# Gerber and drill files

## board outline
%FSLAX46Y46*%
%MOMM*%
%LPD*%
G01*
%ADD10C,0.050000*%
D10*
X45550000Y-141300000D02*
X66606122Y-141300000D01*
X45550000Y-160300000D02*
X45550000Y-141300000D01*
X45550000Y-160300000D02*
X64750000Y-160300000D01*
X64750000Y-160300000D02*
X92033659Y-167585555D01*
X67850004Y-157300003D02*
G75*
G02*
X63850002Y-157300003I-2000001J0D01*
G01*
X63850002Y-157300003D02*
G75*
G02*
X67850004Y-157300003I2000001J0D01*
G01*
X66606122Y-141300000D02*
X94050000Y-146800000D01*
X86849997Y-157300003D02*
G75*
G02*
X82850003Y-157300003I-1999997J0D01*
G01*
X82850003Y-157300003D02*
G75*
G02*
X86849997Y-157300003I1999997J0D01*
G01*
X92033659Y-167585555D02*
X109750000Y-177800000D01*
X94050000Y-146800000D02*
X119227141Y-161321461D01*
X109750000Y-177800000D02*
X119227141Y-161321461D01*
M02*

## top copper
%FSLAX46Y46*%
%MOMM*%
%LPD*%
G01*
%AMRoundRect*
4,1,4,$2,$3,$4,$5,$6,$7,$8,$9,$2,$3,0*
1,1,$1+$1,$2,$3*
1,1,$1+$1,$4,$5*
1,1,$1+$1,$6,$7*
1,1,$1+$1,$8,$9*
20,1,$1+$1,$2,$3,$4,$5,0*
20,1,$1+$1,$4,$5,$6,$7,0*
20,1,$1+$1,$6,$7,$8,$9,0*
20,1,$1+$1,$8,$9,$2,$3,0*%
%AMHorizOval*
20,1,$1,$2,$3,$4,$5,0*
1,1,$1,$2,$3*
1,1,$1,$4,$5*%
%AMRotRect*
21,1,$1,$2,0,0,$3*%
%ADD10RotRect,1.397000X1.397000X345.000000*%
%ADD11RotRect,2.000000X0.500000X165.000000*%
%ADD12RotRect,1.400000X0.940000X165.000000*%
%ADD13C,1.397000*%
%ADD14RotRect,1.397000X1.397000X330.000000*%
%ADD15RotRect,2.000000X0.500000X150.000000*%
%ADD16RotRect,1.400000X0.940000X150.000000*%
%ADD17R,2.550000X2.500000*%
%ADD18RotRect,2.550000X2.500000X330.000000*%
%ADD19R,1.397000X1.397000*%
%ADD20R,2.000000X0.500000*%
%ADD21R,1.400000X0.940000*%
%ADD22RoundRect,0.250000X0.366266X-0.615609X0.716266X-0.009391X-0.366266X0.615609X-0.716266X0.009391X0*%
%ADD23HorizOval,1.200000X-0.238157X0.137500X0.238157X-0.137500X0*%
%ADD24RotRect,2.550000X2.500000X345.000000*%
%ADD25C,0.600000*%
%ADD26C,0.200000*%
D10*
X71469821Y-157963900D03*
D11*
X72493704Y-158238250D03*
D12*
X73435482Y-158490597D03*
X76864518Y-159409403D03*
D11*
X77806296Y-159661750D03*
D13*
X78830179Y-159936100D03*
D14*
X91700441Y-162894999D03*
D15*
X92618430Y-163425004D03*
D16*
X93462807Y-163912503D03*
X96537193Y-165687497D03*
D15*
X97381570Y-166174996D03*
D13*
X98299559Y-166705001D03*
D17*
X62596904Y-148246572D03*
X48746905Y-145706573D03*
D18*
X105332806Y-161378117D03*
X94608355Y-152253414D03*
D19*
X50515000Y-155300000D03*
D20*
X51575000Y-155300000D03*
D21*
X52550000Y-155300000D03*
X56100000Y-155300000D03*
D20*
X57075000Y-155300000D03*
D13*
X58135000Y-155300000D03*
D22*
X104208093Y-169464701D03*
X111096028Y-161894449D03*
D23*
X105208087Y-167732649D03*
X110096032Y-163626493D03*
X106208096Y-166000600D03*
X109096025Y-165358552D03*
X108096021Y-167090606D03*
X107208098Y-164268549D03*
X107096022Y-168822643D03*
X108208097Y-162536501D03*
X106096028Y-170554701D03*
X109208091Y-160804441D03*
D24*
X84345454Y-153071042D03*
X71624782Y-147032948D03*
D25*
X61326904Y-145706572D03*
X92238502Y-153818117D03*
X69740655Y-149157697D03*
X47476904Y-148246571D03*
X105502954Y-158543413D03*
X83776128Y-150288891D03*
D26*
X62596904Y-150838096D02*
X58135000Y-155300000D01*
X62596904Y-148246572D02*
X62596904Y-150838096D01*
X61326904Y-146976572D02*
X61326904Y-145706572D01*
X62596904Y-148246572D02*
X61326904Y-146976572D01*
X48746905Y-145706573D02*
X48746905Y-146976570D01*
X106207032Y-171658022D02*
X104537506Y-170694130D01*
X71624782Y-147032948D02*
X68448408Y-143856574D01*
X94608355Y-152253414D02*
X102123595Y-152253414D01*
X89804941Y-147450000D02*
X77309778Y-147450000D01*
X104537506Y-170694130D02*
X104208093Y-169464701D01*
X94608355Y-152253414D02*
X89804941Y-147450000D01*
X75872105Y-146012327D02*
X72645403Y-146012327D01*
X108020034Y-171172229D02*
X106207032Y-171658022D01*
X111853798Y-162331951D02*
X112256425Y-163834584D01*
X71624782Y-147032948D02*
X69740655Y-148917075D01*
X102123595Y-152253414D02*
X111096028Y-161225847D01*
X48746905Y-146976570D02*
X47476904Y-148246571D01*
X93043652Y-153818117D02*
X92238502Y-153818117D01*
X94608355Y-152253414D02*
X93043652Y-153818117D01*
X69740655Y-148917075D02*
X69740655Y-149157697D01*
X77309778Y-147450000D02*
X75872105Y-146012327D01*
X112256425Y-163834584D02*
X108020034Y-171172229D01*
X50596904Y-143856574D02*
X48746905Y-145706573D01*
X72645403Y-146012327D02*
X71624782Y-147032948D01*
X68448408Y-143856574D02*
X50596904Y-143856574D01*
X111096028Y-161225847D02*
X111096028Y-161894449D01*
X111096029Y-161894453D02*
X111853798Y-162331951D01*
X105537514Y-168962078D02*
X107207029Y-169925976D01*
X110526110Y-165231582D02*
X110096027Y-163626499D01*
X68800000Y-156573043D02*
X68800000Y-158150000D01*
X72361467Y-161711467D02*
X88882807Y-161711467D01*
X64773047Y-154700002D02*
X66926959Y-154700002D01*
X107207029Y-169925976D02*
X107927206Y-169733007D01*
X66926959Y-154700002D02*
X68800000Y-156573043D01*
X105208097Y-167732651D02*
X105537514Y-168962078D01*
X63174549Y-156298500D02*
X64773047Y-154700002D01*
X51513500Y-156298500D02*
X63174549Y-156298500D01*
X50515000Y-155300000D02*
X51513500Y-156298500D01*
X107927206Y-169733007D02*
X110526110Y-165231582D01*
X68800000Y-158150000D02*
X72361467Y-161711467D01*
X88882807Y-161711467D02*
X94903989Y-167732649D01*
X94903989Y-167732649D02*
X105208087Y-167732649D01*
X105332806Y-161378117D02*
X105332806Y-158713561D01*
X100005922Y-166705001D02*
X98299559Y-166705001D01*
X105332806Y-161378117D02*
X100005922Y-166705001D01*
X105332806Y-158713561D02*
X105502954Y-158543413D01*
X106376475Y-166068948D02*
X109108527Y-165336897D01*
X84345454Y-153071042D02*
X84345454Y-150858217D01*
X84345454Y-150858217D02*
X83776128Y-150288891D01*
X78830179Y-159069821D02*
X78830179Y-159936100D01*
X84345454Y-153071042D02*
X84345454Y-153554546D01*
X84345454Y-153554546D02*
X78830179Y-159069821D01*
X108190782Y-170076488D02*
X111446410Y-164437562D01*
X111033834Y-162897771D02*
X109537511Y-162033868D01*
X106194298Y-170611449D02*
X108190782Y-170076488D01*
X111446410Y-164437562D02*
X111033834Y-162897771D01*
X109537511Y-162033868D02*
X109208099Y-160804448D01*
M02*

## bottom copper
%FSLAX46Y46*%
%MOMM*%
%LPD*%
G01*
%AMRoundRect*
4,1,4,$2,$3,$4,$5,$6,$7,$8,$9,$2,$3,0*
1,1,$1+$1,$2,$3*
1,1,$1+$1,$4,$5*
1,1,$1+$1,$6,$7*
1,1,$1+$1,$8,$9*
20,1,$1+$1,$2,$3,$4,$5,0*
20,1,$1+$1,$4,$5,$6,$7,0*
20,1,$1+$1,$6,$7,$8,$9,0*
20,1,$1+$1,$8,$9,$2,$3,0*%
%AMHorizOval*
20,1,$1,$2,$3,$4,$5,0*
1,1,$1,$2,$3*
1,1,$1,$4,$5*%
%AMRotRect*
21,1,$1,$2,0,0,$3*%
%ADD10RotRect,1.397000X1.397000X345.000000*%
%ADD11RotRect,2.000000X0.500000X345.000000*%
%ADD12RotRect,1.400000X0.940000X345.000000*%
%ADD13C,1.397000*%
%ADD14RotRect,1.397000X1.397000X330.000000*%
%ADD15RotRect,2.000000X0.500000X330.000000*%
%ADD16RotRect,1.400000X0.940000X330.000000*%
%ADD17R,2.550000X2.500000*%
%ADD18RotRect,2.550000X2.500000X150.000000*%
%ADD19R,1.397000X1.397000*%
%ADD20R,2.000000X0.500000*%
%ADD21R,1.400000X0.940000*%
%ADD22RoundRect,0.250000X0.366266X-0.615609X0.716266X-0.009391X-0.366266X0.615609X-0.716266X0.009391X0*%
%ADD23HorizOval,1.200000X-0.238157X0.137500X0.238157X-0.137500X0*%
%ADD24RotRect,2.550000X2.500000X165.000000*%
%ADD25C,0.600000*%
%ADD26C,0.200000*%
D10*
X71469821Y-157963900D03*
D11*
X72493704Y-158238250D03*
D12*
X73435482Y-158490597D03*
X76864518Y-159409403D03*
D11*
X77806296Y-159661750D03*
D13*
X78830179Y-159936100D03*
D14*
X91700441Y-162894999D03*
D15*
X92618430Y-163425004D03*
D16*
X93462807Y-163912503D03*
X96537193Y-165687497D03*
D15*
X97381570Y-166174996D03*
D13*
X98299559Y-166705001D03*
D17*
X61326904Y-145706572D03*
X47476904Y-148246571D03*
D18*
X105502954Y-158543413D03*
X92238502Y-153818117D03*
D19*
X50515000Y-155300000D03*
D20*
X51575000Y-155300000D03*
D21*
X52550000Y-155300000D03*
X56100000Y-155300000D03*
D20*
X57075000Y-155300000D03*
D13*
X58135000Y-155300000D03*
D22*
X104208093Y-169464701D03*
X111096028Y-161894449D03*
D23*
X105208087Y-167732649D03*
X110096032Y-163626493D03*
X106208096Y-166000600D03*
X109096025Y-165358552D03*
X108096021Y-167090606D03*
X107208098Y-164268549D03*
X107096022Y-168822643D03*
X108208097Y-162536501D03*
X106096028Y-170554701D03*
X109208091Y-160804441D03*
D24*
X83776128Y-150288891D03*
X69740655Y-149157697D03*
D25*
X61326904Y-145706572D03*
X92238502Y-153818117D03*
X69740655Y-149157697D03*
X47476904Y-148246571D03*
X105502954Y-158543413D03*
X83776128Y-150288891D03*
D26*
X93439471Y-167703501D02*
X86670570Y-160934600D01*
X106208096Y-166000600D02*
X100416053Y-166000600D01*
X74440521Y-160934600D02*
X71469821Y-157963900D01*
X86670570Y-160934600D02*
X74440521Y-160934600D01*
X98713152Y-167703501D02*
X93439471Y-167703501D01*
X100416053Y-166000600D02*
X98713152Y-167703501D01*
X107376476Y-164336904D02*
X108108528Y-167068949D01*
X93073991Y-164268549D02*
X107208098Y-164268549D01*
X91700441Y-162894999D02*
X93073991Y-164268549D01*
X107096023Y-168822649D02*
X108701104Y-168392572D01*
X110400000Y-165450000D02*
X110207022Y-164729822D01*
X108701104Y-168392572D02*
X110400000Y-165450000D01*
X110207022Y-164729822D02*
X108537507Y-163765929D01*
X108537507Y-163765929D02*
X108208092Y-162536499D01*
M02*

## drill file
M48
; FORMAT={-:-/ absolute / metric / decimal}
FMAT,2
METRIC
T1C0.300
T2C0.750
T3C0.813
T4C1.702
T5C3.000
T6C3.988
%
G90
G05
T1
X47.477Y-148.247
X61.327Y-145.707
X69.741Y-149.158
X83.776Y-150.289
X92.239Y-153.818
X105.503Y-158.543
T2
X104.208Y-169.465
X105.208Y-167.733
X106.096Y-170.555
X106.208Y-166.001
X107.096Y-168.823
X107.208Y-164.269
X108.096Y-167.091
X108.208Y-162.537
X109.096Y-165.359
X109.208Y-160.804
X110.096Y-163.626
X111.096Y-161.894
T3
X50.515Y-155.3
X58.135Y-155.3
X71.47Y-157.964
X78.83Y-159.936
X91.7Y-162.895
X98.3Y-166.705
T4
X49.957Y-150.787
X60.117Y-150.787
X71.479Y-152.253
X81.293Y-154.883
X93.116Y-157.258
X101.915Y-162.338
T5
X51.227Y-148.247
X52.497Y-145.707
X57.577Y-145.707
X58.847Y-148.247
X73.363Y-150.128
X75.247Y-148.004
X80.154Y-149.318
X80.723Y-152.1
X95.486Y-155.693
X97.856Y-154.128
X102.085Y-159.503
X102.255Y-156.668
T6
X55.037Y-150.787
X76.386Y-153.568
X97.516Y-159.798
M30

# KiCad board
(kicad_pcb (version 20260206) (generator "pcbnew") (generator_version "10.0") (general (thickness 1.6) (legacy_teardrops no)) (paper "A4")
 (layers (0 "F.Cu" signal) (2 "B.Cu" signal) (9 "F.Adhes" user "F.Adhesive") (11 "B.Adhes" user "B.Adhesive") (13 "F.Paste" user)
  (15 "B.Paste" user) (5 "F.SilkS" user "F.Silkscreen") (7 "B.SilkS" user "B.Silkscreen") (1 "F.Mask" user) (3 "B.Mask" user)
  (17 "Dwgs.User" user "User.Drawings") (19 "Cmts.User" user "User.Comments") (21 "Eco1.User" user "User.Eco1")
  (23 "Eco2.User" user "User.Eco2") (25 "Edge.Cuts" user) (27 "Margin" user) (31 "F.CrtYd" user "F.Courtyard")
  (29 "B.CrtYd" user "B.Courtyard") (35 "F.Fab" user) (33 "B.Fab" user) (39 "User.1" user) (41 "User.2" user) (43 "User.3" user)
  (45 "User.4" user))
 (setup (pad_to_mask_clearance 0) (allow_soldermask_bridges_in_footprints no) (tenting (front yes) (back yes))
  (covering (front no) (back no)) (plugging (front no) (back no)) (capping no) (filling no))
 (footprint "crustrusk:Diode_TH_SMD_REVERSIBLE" (layer "F.Cu") (at 75.15 158.95 -15)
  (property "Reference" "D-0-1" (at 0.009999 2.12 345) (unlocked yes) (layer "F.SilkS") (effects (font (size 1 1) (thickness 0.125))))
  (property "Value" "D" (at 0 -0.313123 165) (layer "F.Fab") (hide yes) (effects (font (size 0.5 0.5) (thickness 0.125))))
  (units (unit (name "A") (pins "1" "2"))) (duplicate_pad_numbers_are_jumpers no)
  (pad "1" thru_hole rect (at -3.810001 0.000001 345) (size 1.397 1.397) (drill 0.8128) (layers "*.Cu" "*.Mask") (remove_unused_layers no)
   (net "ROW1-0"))
  (pad "1" smd rect (at -2.749999 0.000002 165) (size 2 0.5) (layers "F.Cu") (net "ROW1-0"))
  (pad "1" smd rect (at -2.749999 0.000002 345) (size 2 0.5) (layers "B.Cu") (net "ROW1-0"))
  (pad "1" smd rect (at -1.774999 0.000001 165) (size 1.4 0.94) (layers "F.Cu" "F.Mask" "F.Paste") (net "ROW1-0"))
  (pad "1" smd rect (at -1.774999 0.000001 345) (size 1.4 0.94) (layers "B.Cu" "B.Mask" "B.Paste") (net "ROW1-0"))
  (pad "2" smd rect (at 1.774999 -0.000001 165) (size 1.4 0.94) (layers "F.Cu" "F.Mask" "F.Paste") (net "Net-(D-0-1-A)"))
  (pad "2" smd rect (at 1.774999 -0.000001 345) (size 1.4 0.94) (layers "B.Cu" "B.Mask" "B.Paste") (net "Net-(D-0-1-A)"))
  (pad "2" smd rect (at 2.749999 -0.000002 165) (size 2 0.5) (layers "F.Cu") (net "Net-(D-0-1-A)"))
  (pad "2" smd rect (at 2.749999 -0.000002 345) (size 2 0.5) (layers "B.Cu") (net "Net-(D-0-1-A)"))
  (pad "2" thru_hole circle (at 3.810001 -0.000001 345) (size 1.397 1.397) (drill 0.8128) (layers "*.Cu" "*.Mask") (remove_unused_layers no)
   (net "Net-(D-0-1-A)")))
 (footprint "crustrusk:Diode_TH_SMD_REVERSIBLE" (layer "F.Cu") (at 95 164.8 -30)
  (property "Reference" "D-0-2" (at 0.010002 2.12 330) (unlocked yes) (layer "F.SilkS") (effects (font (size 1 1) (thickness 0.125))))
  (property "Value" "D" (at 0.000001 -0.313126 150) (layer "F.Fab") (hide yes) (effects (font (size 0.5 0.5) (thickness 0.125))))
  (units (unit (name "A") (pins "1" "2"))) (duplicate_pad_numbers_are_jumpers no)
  (pad "1" thru_hole rect (at -3.810002 0 330) (size 1.397 1.397) (drill 0.8128) (layers "*.Cu" "*.Mask") (remove_unused_layers no)
   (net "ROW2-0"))
  (pad "1" smd rect (at -2.749998 0.000004 150) (size 2 0.5) (layers "F.Cu") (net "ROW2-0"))
  (pad "1" smd rect (at -2.749998 0.000004 330) (size 2 0.5) (layers "B.Cu") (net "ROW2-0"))
  (pad "1" smd rect (at -1.774997 0.000002 150) (size 1.4 0.94) (layers "F.Cu" "F.Mask" "F.Paste") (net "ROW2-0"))
  (pad "1" smd rect (at -1.774997 0.000002 330) (size 1.4 0.94) (layers "B.Cu" "B.Mask" "B.Paste") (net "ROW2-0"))
  (pad "2" smd rect (at 1.774997 -0.000002 150) (size 1.4 0.94) (layers "F.Cu" "F.Mask" "F.Paste") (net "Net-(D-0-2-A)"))
  (pad "2" smd rect (at 1.774997 -0.000002 330) (size 1.4 0.94) (layers "B.Cu" "B.Mask" "B.Paste") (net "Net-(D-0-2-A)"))
  (pad "2" smd rect (at 2.749998 -0.000004 150) (size 2 0.5) (layers "F.Cu") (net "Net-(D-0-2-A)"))
  (pad "2" smd rect (at 2.749998 -0.000004 330) (size 2 0.5) (layers "B.Cu") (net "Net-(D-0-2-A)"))
  (pad "2" thru_hole circle (at 3.810002 0 330) (size 1.397 1.397) (drill 0.8128) (layers "*.Cu" "*.Mask") (remove_unused_layers no)
   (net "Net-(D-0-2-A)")))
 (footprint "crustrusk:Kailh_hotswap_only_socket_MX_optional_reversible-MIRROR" (layer "F.Cu") (at 55.036904 150.786572)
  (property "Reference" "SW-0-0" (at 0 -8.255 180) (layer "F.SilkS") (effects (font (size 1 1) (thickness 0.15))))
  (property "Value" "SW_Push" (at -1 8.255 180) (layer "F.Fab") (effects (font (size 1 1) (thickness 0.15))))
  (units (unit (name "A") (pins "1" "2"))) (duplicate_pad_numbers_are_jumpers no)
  (pad "" np_thru_hole circle (at -5.08 0) (size 1.7018 1.7018) (drill 1.7018) (layers "*.Cu" "*.Mask"))
  (pad "" np_thru_hole circle (at -3.81 -2.54 180) (size 3 3) (drill 3) (layers "*.Cu" "*.Mask"))
  (pad "" np_thru_hole circle (at -2.54 -5.079998) (size 3 3) (drill 3) (layers "*.Cu" "*.Mask"))
  (pad "" np_thru_hole circle (at 0 0) (size 3.9878 3.9878) (drill 3.9878) (layers "*.Cu" "*.Mask"))
  (pad "" np_thru_hole circle (at 2.540002 -5.080001 180) (size 3 3) (drill 3) (layers "*.Cu" "*.Mask"))
  (pad "" np_thru_hole circle (at 3.81 -2.54) (size 3 3) (drill 3) (layers "*.Cu" "*.Mask"))
  (pad "" np_thru_hole circle (at 5.08 0) (size 1.7018 1.7018) (drill 1.7018) (layers "*.Cu" "*.Mask"))
  (pad "1" smd rect (at 6.29 -5.08 180) (size 2.55 2.5) (layers "B.Cu" "B.Mask" "B.Paste") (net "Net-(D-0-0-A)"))
  (pad "1" smd rect (at 7.56 -2.54) (size 2.55 2.5) (layers "F.Cu" "F.Mask" "F.Paste") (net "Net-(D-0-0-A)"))
  (pad "2" smd rect (at -7.56 -2.540001 180) (size 2.55 2.5) (layers "B.Cu" "B.Mask" "B.Paste") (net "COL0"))
  (pad "2" smd rect (at -6.289999 -5.079999) (size 2.55 2.5) (layers "F.Cu" "F.Mask" "F.Paste") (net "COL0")))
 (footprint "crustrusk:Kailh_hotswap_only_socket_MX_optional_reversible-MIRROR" (layer "F.Cu") (at 97.515654 159.797822 -30)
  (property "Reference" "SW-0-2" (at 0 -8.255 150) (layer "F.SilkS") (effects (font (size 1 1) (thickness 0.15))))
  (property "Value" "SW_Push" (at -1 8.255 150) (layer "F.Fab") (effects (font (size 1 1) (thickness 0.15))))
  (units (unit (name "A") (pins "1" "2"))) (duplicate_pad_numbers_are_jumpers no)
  (pad "" np_thru_hole circle (at -5.08 0 330) (size 1.7018 1.7018) (drill 1.7018) (layers "*.Cu" "*.Mask"))
  (pad "" np_thru_hole circle (at -3.81 -2.54 150) (size 3 3) (drill 3) (layers "*.Cu" "*.Mask"))
  (pad "" np_thru_hole circle (at -2.54 -5.079997 330) (size 3 3) (drill 3) (layers "*.Cu" "*.Mask"))
  (pad "" np_thru_hole circle (at 0 0 330) (size 3.9878 3.9878) (drill 3.9878) (layers "*.Cu" "*.Mask"))
  (pad "" np_thru_hole circle (at 2.540002 -5.080001 150) (size 3 3) (drill 3) (layers "*.Cu" "*.Mask"))
  (pad "" np_thru_hole circle (at 3.81 -2.540001 330) (size 3 3) (drill 3) (layers "*.Cu" "*.Mask"))
  (pad "" np_thru_hole circle (at 5.08 0 330) (size 1.7018 1.7018) (drill 1.7018) (layers "*.Cu" "*.Mask"))
  (pad "1" smd rect (at 6.29 -5.08 150) (size 2.55 2.5) (layers "B.Cu" "B.Mask" "B.Paste") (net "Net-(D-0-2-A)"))
  (pad "1" smd rect (at 7.56 -2.54 330) (size 2.55 2.5) (layers "F.Cu" "F.Mask" "F.Paste") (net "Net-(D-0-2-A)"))
  (pad "2" smd rect (at -7.56 -2.54 150) (size 2.55 2.5) (layers "B.Cu" "B.Mask" "B.Paste") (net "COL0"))
  (pad "2" smd rect (at -6.289999 -5.079999 330) (size 2.55 2.5) (layers "F.Cu" "F.Mask" "F.Paste") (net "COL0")))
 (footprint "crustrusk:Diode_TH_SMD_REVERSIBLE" (layer "F.Cu") (at 54.325 155.3)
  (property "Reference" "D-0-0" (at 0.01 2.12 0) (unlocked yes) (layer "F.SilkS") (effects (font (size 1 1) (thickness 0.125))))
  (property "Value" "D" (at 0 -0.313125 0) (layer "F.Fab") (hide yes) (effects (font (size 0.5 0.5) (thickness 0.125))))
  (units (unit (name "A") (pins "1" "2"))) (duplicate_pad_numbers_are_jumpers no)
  (pad "1" thru_hole rect (at -3.81 0) (size 1.397 1.397) (drill 0.8128) (layers "*.Cu" "*.Mask") (remove_unused_layers no) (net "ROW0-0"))
  (pad "1" smd rect (at -2.75 0 180) (size 2 0.5) (layers "F.Cu") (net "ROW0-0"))
  (pad "1" smd rect (at -2.75 0) (size 2 0.5) (layers "B.Cu") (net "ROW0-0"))
  (pad "1" smd rect (at -1.775 0 180) (size 1.4 0.94) (layers "F.Cu" "F.Mask" "F.Paste") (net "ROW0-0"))
  (pad "1" smd rect (at -1.775 0) (size 1.4 0.94) (layers "B.Cu" "B.Mask" "B.Paste") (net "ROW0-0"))
  (pad "2" smd rect (at 1.775 0 180) (size 1.4 0.94) (layers "F.Cu" "F.Mask" "F.Paste") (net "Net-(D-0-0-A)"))
  (pad "2" smd rect (at 1.775 0) (size 1.4 0.94) (layers "B.Cu" "B.Mask" "B.Paste") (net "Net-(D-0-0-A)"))
  (pad "2" smd rect (at 2.75 0 180) (size 2 0.5) (layers "F.Cu") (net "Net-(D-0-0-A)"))
  (pad "2" smd rect (at 2.75 0) (size 2 0.5) (layers "B.Cu") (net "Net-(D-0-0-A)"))
  (pad "2" thru_hole circle (at 3.81 0) (size 1.397 1.397) (drill 0.8128) (layers "*.Cu" "*.Mask") (remove_unused_layers no)
   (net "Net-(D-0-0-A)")))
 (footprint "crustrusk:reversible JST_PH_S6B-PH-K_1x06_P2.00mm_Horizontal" (layer "F.Cu") (at 104.208093 169.464701 60)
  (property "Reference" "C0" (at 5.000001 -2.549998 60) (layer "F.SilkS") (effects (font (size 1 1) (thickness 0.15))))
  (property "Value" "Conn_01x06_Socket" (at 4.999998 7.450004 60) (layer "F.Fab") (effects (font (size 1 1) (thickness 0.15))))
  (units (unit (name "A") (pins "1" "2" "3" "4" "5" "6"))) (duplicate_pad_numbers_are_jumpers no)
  (pad "1" thru_hole roundrect (at 0 0 60) (size 1.2 1.75) (drill 0.75) (layers "*.Cu" "*.Mask") (remove_unused_layers no)
   (roundrect_rratio 0.208333) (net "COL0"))
  (pad "1" thru_hole roundrect (at 9.999998 2.180001 60) (size 1.2 1.75) (drill 0.75) (layers "*.Cu" "*.Mask") (remove_unused_layers no)
   (roundrect_rratio 0.208333) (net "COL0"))
  (pad "2" thru_hole oval (at 1.999998 -0.000006 60) (size 1.2 1.75) (drill 0.75) (layers "*.Cu" "*.Mask") (remove_unused_layers no)
   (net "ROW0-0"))
  (pad "2" thru_hole oval (at 8.000006 2.180001 60) (size 1.2 1.75) (drill 0.75) (layers "*.Cu" "*.Mask") (remove_unused_layers no)
   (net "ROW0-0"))
  (pad "3" thru_hole oval (at 4.000001 0.000003 60) (size 1.2 1.75) (drill 0.75) (layers "*.Cu" "*.Mask") (remove_unused_layers no)
   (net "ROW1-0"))
  (pad "3" thru_hole oval (at 5.999995 2.179999 60) (size 1.2 1.75) (drill 0.75) (layers "*.Cu" "*.Mask") (remove_unused_layers no)
   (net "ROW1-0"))
  (pad "4" thru_hole oval (at 3.999991 2.179997 60) (size 1.2 1.75) (drill 0.75) (layers "*.Cu" "*.Mask") (remove_unused_layers no)
   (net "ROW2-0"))
  (pad "4" thru_hole oval (at 6.000002 0.000005 60) (size 1.2 1.75) (drill 0.75) (layers "*.Cu" "*.Mask") (remove_unused_layers no)
   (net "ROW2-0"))
  (pad "5" thru_hole oval (at 2.000003 2.179991 60) (size 1.2 1.75) (drill 0.75) (layers "*.Cu" "*.Mask") (remove_unused_layers no)
   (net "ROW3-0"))
  (pad "5" thru_hole oval (at 7.999999 0.000005 60) (size 1.2 1.75) (drill 0.75) (layers "*.Cu" "*.Mask") (remove_unused_layers no)
   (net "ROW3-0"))
  (pad "6" thru_hole oval (at 0 2.18 60) (size 1.2 1.75) (drill 0.75) (layers "*.Cu" "*.Mask") (remove_unused_layers no) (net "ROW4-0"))
  (pad "6" thru_hole oval (at 10.000004 -0.000005 60) (size 1.2 1.75) (drill 0.75) (layers "*.Cu" "*.Mask") (remove_unused_layers no)
   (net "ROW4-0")))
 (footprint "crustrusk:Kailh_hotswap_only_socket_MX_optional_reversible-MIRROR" (layer "F.Cu") (at 76.385654 153.567822 -15)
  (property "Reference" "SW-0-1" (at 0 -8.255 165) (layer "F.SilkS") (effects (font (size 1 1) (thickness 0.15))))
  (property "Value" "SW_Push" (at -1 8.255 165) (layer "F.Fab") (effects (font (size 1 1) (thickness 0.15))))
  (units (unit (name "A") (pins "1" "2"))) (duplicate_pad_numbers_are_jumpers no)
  (pad "" np_thru_hole circle (at -5.08 0 345) (size 1.7018 1.7018) (drill 1.7018) (layers "*.Cu" "*.Mask"))
  (pad "" np_thru_hole circle (at -3.81 -2.54 165) (size 3 3) (drill 3) (layers "*.Cu" "*.Mask"))
  (pad "" np_thru_hole circle (at -2.54 -5.079998 345) (size 3 3) (drill 3) (layers "*.Cu" "*.Mask"))
  (pad "" np_thru_hole circle (at 0 0 345) (size 3.9878 3.9878) (drill 3.9878) (layers "*.Cu" "*.Mask"))
  (pad "" np_thru_hole circle (at 2.540003 -5.080001 165) (size 3 3) (drill 3) (layers "*.Cu" "*.Mask"))
  (pad "" np_thru_hole circle (at 3.81 -2.54 345) (size 3 3) (drill 3) (layers "*.Cu" "*.Mask"))
  (pad "" np_thru_hole circle (at 5.08 0 345) (size 1.7018 1.7018) (drill 1.7018) (layers "*.Cu" "*.Mask"))
  (pad "1" smd rect (at 6.29 -5.08 165) (size 2.55 2.5) (layers "B.Cu" "B.Mask" "B.Paste") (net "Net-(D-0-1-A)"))
  (pad "1" smd rect (at 7.56 -2.54 345) (size 2.55 2.5) (layers "F.Cu" "F.Mask" "F.Paste") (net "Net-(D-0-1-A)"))
  (pad "2" smd rect (at -7.56 -2.540001 165) (size 2.55 2.5) (layers "B.Cu" "B.Mask" "B.Paste") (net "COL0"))
  (pad "2" smd rect (at -6.289999 -5.079999 345) (size 2.55 2.5) (layers "F.Cu" "F.Mask" "F.Paste") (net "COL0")))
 (gr_line (start 45.55 141.3) (end 66.606122 141.3) (stroke (width 0.05) (type default)) (layer "Edge.Cuts"))
 (gr_line (start 45.55 160.3) (end 45.55 141.3) (stroke (width 0.05) (type default)) (layer "Edge.Cuts"))
 (gr_line (start 45.55 160.3) (end 64.75 160.3) (stroke (width 0.05) (type default)) (layer "Edge.Cuts"))
 (gr_line (start 64.75 160.3) (end 92.033659 167.585555) (stroke (width 0.05) (type default)) (layer "Edge.Cuts"))
 (gr_circle (center 65.850003 157.300003) (end 63.850002 157.300003) (stroke (width 0.05) (type default)) (fill no) (layer "Edge.Cuts"))
 (gr_line (start 66.606122 141.3) (end 94.05 146.8) (stroke (width 0.05) (type default)) (layer "Edge.Cuts"))
 (gr_circle (center 84.85 157.300003) (end 82.850003 157.300003) (stroke (width 0.05) (type default)) (fill no) (layer "Edge.Cuts"))
 (gr_line (start 92.033659 167.585555) (end 109.75 177.8) (stroke (width 0.05) (type default)) (layer "Edge.Cuts"))
 (gr_line (start 94.05 146.8) (end 119.227141 161.321461) (stroke (width 0.05) (type default)) (layer "Edge.Cuts"))
 (gr_line (start 109.75 177.8) (end 119.227141 161.321461) (stroke (width 0.05) (type default)) (layer "Edge.Cuts"))
 (segment (start 62.596904 150.838096) (end 58.135 155.3) (width 0.2) (layer "F.Cu") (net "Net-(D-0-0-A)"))
 (segment (start 62.596904 148.246572) (end 62.596904 150.838096) (width 0.2) (layer "F.Cu") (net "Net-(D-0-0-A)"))
 (segment (start 61.326904 146.976572) (end 61.326904 145.706572) (width 0.2) (layer "F.Cu") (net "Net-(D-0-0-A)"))
 (segment (start 62.596904 148.246572) (end 61.326904 146.976572) (width 0.2) (layer "F.Cu") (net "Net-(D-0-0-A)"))
 (via (at 61.326904 145.706572) (size 0.6) (drill 0.3) (layers "F.Cu" "B.Cu") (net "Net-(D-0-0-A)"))
 (segment (start 48.746905 145.706573) (end 48.746905 146.97657) (width 0.2) (layer "F.Cu") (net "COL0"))
 (segment (start 106.207032 171.658022) (end 104.537506 170.69413) (width 0.2) (layer "F.Cu") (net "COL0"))
 (segment (start 71.624782 147.032948) (end 68.448408 143.856574) (width 0.2) (layer "F.Cu") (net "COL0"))
 (segment (start 94.608355 152.253414) (end 102.123595 152.253414) (width 0.2) (layer "F.Cu") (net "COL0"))
 (segment (start 89.804941 147.45) (end 77.309778 147.45) (width 0.2) (layer "F.Cu") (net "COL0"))
 (segment (start 104.537506 170.69413) (end 104.208093 169.464701) (width 0.2) (layer "F.Cu") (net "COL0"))
 (segment (start 94.608355 152.253414) (end 89.804941 147.45) (width 0.2) (layer "F.Cu") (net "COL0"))
 (segment (start 75.872105 146.012327) (end 72.645403 146.012327) (width 0.2) (layer "F.Cu") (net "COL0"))
 (segment (start 108.020034 171.172229) (end 106.207032 171.658022) (width 0.2) (layer "F.Cu") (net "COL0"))
 (segment (start 111.853798 162.331951) (end 112.256425 163.834584) (width 0.2) (layer "F.Cu") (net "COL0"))
 (segment (start 71.624782 147.032948) (end 69.740655 148.917075) (width 0.2) (layer "F.Cu") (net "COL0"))
 (segment (start 102.123595 152.253414) (end 111.096028 161.225847) (width 0.2) (layer "F.Cu") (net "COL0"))
 (segment (start 48.746905 146.97657) (end 47.476904 148.246571) (width 0.2) (layer "F.Cu") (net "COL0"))
 (segment (start 93.043652 153.818117) (end 92.238502 153.818117) (width 0.2) (layer "F.Cu") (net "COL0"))
 (segment (start 94.608355 152.253414) (end 93.043652 153.818117) (width 0.2) (layer "F.Cu") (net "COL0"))
 (segment (start 69.740655 148.917075) (end 69.740655 149.157697) (width 0.2) (layer "F.Cu") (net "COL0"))
 (segment (start 77.309778 147.45) (end 75.872105 146.012327) (width 0.2) (layer "F.Cu") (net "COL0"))
 (segment (start 112.256425 163.834584) (end 108.020034 171.172229) (width 0.2) (layer "F.Cu") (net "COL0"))
 (segment (start 50.596904 143.856574) (end 48.746905 145.706573) (width 0.2) (layer "F.Cu") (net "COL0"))
 (segment (start 72.645403 146.012327) (end 71.624782 147.032948) (width 0.2) (layer "F.Cu") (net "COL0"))
 (segment (start 68.448408 143.856574) (end 50.596904 143.856574) (width 0.2) (layer "F.Cu") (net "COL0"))
 (segment (start 111.096028 161.225847) (end 111.096028 161.894449) (width 0.2) (layer "F.Cu") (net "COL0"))
 (segment (start 111.096029 161.894453) (end 111.853798 162.331951) (width 0.2) (layer "F.Cu") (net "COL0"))
 (via (at 92.238502 153.818117) (size 0.6) (drill 0.3) (layers "F.Cu" "B.Cu") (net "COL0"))
 (via (at 69.740655 149.157697) (size 0.6) (drill 0.3) (layers "F.Cu" "B.Cu") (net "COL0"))
 (via (at 47.476904 148.246571) (size 0.6) (drill 0.3) (layers "F.Cu" "B.Cu") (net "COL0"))
 (segment (start 105.537514 168.962078) (end 107.207029 169.925976) (width 0.2) (layer "F.Cu") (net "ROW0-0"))
 (segment (start 110.52611 165.231582) (end 110.096027 163.626499) (width 0.2) (layer "F.Cu") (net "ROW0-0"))
 (segment (start 68.8 156.573043) (end 68.8 158.15) (width 0.2) (layer "F.Cu") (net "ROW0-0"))
 (segment (start 72.361467 161.711467) (end 88.882807 161.711467) (width 0.2) (layer "F.Cu") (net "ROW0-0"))
 (segment (start 64.773047 154.700002) (end 66.926959 154.700002) (width 0.2) (layer "F.Cu") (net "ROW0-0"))
 (segment (start 107.207029 169.925976) (end 107.927206 169.733007) (width 0.2) (layer "F.Cu") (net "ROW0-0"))
 (segment (start 66.926959 154.700002) (end 68.8 156.573043) (width 0.2) (layer "F.Cu") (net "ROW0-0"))
 (segment (start 105.208097 167.732651) (end 105.537514 168.962078) (width 0.2) (layer "F.Cu") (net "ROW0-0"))
 (segment (start 63.174549 156.2985) (end 64.773047 154.700002) (width 0.2) (layer "F.Cu") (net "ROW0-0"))
 (segment (start 51.5135 156.2985) (end 63.174549 156.2985) (width 0.2) (layer "F.Cu") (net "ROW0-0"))
 (segment (start 50.515 155.3) (end 51.5135 156.2985) (width 0.2) (layer "F.Cu") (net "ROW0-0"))
 (segment (start 107.927206 169.733007) (end 110.52611 165.231582) (width 0.2) (layer "F.Cu") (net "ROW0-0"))
 (segment (start 68.8 158.15) (end 72.361467 161.711467) (width 0.2) (layer "F.Cu") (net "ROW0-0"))
 (segment (start 88.882807 161.711467) (end 94.903989 167.732649) (width 0.2) (layer "F.Cu") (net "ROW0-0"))
 (segment (start 94.903989 167.732649) (end 105.208087 167.732649) (width 0.2) (layer "F.Cu") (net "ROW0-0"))
 (segment (start 105.332806 161.378117) (end 105.332806 158.713561) (width 0.2) (layer "F.Cu") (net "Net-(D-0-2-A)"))
 (segment (start 100.005922 166.705001) (end 98.299559 166.705001) (width 0.2) (layer "F.Cu") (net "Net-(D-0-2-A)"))
 (segment (start 105.332806 161.378117) (end 100.005922 166.705001) (width 0.2) (layer "F.Cu") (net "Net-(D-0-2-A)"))
 (segment (start 105.332806 158.713561) (end 105.502954 158.543413) (width 0.2) (layer "F.Cu") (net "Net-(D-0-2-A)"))
 (via (at 105.502954 158.543413) (size 0.6) (drill 0.3) (layers "F.Cu" "B.Cu") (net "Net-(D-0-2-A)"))
 (segment (start 106.376475 166.068948) (end 109.108527 165.336897) (width 0.2) (layer "F.Cu") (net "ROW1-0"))
 (segment (start 93.439471 167.703501) (end 86.67057 160.9346) (width 0.2) (layer "B.Cu") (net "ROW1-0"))
 (segment (start 106.208096 166.0006) (end 100.416053 166.0006) (width 0.2) (layer "B.Cu") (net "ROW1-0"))
 (segment (start 74.440521 160.9346) (end 71.469821 157.9639) (width 0.2) (layer "B.Cu") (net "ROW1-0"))
 (segment (start 86.67057 160.9346) (end 74.440521 160.9346) (width 0.2) (layer "B.Cu") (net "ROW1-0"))
 (segment (start 98.713152 167.703501) (end 93.439471 167.703501) (width 0.2) (layer "B.Cu") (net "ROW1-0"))
 (segment (start 100.416053 166.0006) (end 98.713152 167.703501) (width 0.2) (layer "B.Cu") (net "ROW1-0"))
 (segment (start 84.345454 153.071042) (end 84.345454 150.858217) (width 0.2) (layer "F.Cu") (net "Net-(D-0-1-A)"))
 (segment (start 84.345454 150.858217) (end 83.776128 150.288891) (width 0.2) (layer "F.Cu") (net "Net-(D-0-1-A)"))
 (segment (start 78.830179 159.069821) (end 78.830179 159.9361) (width 0.2) (layer "F.Cu") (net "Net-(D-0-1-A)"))
 (segment (start 84.345454 153.071042) (end 84.345454 153.554546) (width 0.2) (layer "F.Cu") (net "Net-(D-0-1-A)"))
 (segment (start 84.345454 153.554546) (end 78.830179 159.069821) (width 0.2) (layer "F.Cu") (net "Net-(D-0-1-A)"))
 (via (at 83.776128 150.288891) (size 0.6) (drill 0.3) (layers "F.Cu" "B.Cu") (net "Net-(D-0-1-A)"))
 (segment (start 107.376476 164.336904) (end 108.108528 167.068949) (width 0.2) (layer "B.Cu") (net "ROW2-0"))
 (segment (start 93.073991 164.268549) (end 107.208098 164.268549) (width 0.2) (layer "B.Cu") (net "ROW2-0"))
 (segment (start 91.700441 162.894999) (end 93.073991 164.268549) (width 0.2) (layer "B.Cu") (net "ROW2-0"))
 (segment (start 107.096023 168.822649) (end 108.701104 168.392572) (width 0.2) (layer "B.Cu") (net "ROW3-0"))
 (segment (start 110.4 165.45) (end 110.207022 164.729822) (width 0.2) (layer "B.Cu") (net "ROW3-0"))
 (segment (start 108.701104 168.392572) (end 110.4 165.45) (width 0.2) (layer "B.Cu") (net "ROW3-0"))
 (segment (start 110.207022 164.729822) (end 108.537507 163.765929) (width 0.2) (layer "B.Cu") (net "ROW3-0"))
 (segment (start 108.537507 163.765929) (end 108.208092 162.536499) (width 0.2) (layer "B.Cu") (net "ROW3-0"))
 (segment (start 108.190782 170.076488) (end 111.44641 164.437562) (width 0.2) (layer "F.Cu") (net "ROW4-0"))
 (segment (start 111.033834 162.897771) (end 109.537511 162.033868) (width 0.2) (layer "F.Cu") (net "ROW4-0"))
 (segment (start 106.194298 170.611449) (end 108.190782 170.076488) (width 0.2) (layer "F.Cu") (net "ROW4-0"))
 (segment (start 111.44641 164.437562) (end 111.033834 162.897771) (width 0.2) (layer "F.Cu") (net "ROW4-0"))
 (segment (start 109.537511 162.033868) (end 109.208099 160.804448) (width 0.2) (layer "F.Cu") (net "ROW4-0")))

